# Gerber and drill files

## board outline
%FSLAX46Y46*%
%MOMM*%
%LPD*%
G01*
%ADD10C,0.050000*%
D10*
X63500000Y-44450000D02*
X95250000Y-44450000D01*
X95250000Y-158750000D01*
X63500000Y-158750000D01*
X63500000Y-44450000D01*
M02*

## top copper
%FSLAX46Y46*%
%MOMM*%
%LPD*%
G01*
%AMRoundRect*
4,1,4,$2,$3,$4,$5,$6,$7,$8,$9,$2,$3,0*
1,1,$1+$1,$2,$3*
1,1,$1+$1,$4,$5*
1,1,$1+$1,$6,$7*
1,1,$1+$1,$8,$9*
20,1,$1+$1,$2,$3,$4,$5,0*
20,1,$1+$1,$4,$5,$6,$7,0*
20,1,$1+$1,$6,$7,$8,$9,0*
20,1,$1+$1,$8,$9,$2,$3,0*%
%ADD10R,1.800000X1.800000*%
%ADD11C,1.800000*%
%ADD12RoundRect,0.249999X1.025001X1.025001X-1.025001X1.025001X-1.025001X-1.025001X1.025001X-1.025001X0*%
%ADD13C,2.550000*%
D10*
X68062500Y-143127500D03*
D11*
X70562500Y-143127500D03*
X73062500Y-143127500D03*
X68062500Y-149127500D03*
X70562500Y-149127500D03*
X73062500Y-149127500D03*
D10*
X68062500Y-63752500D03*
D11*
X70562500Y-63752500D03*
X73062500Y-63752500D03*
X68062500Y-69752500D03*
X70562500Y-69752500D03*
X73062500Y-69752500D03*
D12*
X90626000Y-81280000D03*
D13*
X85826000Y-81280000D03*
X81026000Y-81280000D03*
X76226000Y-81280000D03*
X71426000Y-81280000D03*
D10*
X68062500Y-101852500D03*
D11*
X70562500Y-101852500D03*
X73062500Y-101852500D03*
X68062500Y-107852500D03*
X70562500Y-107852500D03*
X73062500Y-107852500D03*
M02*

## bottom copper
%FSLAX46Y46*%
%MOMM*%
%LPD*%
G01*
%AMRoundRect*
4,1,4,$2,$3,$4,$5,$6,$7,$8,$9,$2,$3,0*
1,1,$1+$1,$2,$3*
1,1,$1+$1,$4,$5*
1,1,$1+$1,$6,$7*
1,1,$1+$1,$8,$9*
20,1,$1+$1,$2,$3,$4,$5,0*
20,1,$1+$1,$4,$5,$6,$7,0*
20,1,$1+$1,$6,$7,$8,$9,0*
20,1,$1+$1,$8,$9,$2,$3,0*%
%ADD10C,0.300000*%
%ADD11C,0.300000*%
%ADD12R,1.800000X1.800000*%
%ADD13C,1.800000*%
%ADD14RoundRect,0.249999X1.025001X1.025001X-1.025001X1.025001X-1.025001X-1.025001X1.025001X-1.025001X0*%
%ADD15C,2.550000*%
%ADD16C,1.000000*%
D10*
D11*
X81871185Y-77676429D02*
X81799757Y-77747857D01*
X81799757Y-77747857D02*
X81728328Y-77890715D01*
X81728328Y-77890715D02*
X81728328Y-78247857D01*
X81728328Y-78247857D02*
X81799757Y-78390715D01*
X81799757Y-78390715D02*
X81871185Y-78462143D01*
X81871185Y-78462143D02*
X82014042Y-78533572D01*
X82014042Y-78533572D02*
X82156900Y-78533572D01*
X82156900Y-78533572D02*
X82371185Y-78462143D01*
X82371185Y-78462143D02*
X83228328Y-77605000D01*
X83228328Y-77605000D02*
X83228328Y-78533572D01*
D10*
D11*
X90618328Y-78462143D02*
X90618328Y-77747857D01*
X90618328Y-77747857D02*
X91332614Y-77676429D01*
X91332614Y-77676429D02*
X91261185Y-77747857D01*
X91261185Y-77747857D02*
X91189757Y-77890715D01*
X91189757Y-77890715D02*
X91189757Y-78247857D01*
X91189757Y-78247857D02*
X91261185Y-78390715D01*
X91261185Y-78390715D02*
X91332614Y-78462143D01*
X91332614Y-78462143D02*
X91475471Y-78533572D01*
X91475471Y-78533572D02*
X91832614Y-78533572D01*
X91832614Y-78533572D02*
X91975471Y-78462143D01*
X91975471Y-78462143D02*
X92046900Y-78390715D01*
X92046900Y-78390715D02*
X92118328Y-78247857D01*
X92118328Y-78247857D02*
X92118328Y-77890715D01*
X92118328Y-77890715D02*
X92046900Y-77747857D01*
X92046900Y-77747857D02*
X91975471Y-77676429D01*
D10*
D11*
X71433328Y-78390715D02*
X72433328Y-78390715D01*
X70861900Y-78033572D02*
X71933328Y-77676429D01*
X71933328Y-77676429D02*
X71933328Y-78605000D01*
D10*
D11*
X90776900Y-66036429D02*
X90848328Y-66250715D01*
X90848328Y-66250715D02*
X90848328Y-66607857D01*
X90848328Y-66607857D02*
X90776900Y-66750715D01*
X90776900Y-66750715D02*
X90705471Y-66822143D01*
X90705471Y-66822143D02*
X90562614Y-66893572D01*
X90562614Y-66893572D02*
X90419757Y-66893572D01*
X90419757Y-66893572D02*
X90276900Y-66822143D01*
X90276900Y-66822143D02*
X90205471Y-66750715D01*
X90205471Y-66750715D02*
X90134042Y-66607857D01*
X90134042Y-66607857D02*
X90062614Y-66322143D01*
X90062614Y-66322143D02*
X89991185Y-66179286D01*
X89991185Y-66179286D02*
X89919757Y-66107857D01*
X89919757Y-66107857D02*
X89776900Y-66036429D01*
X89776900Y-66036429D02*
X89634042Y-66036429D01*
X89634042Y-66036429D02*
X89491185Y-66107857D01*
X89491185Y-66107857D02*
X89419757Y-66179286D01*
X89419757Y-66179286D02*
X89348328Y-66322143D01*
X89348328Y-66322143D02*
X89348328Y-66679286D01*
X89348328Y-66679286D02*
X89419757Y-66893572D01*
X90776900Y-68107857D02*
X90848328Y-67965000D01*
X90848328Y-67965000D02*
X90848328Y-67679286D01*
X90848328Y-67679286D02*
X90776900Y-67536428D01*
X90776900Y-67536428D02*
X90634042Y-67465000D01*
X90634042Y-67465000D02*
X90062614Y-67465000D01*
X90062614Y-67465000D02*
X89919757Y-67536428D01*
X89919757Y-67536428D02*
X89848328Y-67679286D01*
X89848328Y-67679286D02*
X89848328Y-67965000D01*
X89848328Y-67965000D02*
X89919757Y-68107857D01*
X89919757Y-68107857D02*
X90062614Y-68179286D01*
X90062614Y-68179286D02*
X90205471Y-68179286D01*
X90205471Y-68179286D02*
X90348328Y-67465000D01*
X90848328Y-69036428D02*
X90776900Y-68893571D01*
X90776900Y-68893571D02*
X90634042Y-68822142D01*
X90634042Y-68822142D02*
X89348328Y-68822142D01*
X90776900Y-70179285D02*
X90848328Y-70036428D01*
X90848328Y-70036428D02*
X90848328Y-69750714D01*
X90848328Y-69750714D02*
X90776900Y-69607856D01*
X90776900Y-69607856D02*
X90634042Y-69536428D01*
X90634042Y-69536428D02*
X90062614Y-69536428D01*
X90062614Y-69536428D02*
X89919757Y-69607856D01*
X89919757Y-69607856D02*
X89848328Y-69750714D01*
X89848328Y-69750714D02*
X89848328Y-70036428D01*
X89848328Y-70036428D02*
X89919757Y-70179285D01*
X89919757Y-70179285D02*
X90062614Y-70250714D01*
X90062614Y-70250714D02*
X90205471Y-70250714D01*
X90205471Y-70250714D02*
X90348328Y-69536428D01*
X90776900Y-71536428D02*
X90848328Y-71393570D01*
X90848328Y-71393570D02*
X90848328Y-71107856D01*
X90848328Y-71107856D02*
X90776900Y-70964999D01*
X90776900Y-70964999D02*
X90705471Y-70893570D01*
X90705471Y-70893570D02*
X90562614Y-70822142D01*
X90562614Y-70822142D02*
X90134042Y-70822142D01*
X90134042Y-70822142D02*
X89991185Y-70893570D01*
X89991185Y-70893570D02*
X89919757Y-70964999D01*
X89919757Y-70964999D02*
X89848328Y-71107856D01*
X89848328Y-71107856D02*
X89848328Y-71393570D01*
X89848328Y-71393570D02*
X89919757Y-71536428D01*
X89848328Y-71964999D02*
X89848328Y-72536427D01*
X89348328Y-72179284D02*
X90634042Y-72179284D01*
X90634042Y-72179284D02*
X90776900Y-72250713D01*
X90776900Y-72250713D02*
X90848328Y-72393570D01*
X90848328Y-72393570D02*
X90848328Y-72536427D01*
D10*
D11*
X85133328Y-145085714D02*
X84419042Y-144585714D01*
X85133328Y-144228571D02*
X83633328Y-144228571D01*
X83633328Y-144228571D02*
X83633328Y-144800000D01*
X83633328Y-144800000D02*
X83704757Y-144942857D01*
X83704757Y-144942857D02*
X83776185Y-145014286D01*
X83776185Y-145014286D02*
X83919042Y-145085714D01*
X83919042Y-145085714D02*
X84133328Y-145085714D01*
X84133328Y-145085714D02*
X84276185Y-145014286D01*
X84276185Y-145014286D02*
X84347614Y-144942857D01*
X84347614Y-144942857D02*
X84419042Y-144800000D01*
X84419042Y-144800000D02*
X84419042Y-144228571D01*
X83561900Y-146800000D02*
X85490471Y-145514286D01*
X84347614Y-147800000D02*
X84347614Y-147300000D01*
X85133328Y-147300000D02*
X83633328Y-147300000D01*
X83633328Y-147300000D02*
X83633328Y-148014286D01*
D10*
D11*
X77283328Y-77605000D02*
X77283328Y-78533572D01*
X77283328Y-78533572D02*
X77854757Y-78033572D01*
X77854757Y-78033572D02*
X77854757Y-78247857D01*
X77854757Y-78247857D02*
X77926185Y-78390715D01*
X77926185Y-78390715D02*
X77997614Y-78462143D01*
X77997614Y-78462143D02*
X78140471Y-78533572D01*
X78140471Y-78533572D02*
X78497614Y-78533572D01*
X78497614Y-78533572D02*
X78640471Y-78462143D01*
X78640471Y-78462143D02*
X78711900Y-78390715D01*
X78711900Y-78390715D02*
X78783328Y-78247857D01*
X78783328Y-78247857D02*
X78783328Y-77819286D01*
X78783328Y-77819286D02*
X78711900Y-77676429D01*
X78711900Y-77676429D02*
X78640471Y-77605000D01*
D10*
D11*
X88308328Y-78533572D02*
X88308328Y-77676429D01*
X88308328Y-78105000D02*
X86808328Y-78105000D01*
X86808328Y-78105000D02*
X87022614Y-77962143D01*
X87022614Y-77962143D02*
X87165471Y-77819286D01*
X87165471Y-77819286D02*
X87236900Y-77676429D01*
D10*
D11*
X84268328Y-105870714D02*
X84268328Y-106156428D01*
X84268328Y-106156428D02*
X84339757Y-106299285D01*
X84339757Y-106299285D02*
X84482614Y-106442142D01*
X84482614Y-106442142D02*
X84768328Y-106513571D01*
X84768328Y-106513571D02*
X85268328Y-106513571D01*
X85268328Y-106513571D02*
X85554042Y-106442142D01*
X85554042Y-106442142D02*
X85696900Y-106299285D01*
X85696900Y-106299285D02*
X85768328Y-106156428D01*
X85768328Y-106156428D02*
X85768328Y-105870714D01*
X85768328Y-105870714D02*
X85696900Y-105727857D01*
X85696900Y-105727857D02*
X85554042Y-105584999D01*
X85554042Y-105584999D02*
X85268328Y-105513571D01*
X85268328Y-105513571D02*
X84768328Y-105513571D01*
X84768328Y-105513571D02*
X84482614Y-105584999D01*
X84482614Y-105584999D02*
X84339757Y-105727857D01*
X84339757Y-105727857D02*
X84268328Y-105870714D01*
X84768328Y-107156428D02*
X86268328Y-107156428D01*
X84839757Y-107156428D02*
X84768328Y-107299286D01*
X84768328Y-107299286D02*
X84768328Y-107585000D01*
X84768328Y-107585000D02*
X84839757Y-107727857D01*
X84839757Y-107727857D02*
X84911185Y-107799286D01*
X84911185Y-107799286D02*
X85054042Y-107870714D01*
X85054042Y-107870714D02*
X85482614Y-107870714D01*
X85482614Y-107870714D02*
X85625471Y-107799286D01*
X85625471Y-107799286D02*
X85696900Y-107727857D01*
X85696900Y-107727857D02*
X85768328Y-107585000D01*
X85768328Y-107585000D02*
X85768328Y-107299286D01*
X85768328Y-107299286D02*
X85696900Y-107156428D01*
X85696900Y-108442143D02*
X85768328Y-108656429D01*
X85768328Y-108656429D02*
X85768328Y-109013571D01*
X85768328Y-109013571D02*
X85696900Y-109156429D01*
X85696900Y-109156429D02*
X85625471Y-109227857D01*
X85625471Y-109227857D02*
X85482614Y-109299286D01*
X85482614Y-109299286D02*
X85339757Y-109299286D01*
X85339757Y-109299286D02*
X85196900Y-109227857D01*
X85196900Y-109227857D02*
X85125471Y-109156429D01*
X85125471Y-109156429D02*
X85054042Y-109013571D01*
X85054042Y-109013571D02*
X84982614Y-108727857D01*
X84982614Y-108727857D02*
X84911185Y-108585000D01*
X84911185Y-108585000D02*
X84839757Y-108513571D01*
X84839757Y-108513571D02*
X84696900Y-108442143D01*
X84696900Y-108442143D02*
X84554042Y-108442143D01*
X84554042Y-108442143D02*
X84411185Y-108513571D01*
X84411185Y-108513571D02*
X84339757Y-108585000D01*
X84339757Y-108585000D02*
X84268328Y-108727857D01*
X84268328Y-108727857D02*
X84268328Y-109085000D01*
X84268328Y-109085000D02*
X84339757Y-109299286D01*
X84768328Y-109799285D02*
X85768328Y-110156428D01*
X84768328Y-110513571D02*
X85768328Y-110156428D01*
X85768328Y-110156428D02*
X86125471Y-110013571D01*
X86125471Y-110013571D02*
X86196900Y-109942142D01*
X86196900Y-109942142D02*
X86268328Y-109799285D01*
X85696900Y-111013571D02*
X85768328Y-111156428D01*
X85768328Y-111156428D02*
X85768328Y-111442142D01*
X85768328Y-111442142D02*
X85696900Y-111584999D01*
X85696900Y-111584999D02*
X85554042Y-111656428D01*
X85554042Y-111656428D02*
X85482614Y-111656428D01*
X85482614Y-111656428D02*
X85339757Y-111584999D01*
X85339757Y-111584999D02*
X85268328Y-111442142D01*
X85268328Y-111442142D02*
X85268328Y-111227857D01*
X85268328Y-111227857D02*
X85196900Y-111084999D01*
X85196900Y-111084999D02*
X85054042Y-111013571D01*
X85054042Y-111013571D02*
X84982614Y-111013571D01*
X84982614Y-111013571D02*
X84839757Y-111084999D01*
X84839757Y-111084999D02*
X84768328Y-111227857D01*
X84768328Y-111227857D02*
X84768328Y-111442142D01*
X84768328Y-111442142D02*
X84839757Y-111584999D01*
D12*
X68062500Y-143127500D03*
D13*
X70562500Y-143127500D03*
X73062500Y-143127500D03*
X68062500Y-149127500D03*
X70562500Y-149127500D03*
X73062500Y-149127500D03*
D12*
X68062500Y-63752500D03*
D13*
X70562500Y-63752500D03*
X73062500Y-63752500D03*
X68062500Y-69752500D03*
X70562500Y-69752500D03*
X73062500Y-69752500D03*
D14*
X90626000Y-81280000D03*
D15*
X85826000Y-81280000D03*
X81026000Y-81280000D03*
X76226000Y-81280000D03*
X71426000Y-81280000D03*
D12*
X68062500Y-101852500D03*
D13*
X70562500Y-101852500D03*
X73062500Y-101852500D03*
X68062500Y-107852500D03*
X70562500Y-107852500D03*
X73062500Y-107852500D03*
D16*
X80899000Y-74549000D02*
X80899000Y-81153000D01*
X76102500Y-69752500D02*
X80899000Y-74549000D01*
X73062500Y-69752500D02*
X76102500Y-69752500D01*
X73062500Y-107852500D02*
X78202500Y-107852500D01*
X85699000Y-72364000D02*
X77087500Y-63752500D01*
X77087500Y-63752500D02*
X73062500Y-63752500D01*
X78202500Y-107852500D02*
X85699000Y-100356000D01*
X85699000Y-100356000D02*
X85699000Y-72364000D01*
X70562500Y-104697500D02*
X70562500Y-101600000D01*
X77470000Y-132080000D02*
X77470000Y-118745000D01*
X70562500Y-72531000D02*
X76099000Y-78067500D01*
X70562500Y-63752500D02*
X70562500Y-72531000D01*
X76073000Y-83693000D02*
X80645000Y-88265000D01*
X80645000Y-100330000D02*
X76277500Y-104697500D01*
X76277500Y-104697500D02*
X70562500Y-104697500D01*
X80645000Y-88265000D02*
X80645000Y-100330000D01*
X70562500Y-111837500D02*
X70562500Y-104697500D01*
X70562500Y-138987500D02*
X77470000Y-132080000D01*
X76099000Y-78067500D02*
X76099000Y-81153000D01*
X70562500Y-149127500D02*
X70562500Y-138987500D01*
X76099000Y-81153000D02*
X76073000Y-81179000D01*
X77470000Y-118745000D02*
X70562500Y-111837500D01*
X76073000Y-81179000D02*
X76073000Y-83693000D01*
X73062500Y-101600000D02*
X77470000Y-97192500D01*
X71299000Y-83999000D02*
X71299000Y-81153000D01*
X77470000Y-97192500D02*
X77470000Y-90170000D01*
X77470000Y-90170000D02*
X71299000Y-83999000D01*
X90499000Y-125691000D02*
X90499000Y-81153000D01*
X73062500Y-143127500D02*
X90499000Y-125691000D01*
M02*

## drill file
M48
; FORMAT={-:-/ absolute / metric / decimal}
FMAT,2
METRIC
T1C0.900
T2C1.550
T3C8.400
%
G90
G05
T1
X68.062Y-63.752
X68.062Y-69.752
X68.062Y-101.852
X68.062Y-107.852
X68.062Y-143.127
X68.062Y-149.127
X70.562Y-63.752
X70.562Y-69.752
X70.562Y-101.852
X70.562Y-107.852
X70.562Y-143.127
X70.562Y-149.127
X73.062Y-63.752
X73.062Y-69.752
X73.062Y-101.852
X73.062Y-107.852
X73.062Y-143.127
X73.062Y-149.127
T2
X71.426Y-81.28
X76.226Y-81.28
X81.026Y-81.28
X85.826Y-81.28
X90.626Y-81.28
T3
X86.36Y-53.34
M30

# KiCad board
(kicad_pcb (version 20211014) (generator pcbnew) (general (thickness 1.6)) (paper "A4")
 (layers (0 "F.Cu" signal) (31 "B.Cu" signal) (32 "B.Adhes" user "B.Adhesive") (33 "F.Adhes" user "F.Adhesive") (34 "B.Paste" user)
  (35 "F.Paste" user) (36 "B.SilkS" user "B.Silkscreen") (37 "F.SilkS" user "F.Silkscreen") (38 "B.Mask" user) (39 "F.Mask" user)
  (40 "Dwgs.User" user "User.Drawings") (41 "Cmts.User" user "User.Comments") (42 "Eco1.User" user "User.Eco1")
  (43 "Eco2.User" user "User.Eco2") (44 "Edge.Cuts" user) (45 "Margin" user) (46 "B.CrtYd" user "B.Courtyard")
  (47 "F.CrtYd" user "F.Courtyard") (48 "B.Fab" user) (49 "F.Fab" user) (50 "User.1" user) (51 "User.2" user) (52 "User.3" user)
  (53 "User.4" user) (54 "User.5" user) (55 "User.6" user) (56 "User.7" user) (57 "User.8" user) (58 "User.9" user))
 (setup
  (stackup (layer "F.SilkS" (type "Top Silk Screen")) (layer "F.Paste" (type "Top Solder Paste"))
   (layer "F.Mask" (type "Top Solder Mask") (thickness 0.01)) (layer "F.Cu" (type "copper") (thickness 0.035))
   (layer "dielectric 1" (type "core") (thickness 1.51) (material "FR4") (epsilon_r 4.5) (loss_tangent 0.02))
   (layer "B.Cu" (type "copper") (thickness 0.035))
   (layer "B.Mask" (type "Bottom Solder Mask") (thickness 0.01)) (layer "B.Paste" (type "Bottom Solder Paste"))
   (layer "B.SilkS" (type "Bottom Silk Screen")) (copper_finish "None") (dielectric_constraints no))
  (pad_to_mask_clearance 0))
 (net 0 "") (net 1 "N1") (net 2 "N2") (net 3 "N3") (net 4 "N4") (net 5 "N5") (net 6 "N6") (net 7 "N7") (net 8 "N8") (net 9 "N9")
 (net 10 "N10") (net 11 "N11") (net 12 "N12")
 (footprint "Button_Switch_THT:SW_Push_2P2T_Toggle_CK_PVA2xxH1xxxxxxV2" (layer "F.Cu") (at 68.0625 143.1275)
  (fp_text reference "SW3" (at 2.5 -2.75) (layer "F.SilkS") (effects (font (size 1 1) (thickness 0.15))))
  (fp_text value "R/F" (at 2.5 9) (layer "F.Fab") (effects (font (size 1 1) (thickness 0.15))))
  (pad "1" thru_hole rect (at 0 0) (size 1.8 1.8) (drill 0.9) (layers *.Cu *.Mask) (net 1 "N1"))
  (pad "2" thru_hole circle (at 2.5 0) (size 1.8 1.8) (drill 0.9) (layers *.Cu *.Mask) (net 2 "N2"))
  (pad "3" thru_hole circle (at 5 0) (size 1.8 1.8) (drill 0.9) (layers *.Cu *.Mask) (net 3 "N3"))
  (pad "4" thru_hole circle (at 0 6) (size 1.8 1.8) (drill 0.9) (layers *.Cu *.Mask) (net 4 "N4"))
  (pad "5" thru_hole circle (at 2.5 6) (size 1.8 1.8) (drill 0.9) (layers *.Cu *.Mask) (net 2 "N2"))
  (pad "6" thru_hole circle (at 5 6) (size 1.8 1.8) (drill 0.9) (layers *.Cu *.Mask) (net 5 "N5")))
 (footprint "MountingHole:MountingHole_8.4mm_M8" (layer "F.Cu") (at 86.36 53.34)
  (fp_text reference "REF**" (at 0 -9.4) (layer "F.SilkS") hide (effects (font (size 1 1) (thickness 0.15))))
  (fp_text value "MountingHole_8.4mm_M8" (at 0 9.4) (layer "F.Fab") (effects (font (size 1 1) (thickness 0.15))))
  (pad "" np_thru_hole circle (at 0 0) (size 8.4 8.4) (drill 8.4) (layers *.Cu *.Mask)))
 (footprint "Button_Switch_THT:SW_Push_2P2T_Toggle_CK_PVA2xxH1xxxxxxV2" (layer "F.Cu") (at 68.0625 63.7525)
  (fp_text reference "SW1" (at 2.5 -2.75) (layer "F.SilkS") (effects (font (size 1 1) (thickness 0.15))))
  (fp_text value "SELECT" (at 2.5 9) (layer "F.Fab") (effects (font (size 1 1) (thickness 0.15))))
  (pad "1" thru_hole rect (at 0 0) (size 1.8 1.8) (drill 0.9) (layers *.Cu *.Mask) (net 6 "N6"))
  (pad "2" thru_hole circle (at 2.5 0) (size 1.8 1.8) (drill 0.9) (layers *.Cu *.Mask) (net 2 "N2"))
  (pad "3" thru_hole circle (at 5 0) (size 1.8 1.8) (drill 0.9) (layers *.Cu *.Mask) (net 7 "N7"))
  (pad "4" thru_hole circle (at 0 6) (size 1.8 1.8) (drill 0.9) (layers *.Cu *.Mask) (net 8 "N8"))
  (pad "5" thru_hole circle (at 2.5 6) (size 1.8 1.8) (drill 0.9) (layers *.Cu *.Mask) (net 2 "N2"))
  (pad "6" thru_hole circle (at 5 6) (size 1.8 1.8) (drill 0.9) (layers *.Cu *.Mask) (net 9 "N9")))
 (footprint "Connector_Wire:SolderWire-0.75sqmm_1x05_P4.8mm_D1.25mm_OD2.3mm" (layer "F.Cu") (at 90.626 81.28 180)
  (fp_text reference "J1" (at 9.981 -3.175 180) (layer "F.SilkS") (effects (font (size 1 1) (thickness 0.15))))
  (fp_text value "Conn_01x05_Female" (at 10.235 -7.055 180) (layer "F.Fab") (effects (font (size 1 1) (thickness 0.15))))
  (pad "1" thru_hole roundrect (at 0 0 180) (size 2.55 2.55) (drill 1.55) (layers *.Cu *.Mask) (roundrect_rratio 0.098039) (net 3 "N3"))
  (pad "2" thru_hole circle (at 4.8 0 180) (size 2.55 2.55) (drill 1.55) (layers *.Cu *.Mask) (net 7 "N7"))
  (pad "3" thru_hole circle (at 9.6 0 180) (size 2.55 2.55) (drill 1.55) (layers *.Cu *.Mask) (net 9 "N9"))
  (pad "4" thru_hole circle (at 14.4 0 180) (size 2.55 2.55) (drill 1.55) (layers *.Cu *.Mask) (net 2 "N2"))
  (pad "5" thru_hole circle (at 19.2 0 180) (size 2.55 2.55) (drill 1.55) (layers *.Cu *.Mask) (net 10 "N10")))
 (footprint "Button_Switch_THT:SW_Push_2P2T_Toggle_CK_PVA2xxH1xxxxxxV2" (layer "F.Cu") (at 68.0625 101.8525)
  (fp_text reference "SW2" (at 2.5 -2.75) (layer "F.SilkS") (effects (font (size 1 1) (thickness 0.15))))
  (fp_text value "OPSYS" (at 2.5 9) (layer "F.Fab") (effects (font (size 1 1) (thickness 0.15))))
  (pad "1" thru_hole rect (at 0 0) (size 1.8 1.8) (drill 0.9) (layers *.Cu *.Mask) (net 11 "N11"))
  (pad "2" thru_hole circle (at 2.5 0) (size 1.8 1.8) (drill 0.9) (layers *.Cu *.Mask) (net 2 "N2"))
  (pad "3" thru_hole circle (at 5 0) (size 1.8 1.8) (drill 0.9) (layers *.Cu *.Mask) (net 10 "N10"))
  (pad "4" thru_hole circle (at 0 6) (size 1.8 1.8) (drill 0.9) (layers *.Cu *.Mask) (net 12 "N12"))
  (pad "5" thru_hole circle (at 2.5 6) (size 1.8 1.8) (drill 0.9) (layers *.Cu *.Mask) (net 2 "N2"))
  (pad "6" thru_hole circle (at 5 6) (size 1.8 1.8) (drill 0.9) (layers *.Cu *.Mask) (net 7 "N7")))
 (gr_rect (start 63.5 44.45) (end 95.25 158.75) (layer "Edge.Cuts") (width 0.05) (fill none))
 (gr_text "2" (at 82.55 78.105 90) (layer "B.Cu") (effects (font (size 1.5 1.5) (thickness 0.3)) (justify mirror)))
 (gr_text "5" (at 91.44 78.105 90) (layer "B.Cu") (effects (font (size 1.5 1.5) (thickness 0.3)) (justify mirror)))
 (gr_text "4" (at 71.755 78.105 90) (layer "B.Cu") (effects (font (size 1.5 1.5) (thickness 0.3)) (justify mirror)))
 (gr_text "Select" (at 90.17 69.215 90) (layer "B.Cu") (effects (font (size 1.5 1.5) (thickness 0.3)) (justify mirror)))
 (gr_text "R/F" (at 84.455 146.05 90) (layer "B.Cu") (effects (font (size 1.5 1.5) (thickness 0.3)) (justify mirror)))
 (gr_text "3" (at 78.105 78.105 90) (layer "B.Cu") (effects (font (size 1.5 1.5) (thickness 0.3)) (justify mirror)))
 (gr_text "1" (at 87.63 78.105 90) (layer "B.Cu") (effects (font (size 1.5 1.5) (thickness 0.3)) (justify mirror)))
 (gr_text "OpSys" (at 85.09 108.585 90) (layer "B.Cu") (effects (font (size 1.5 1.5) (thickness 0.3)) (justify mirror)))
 (segment (start 80.899 74.549) (end 80.899 81.153) (width 1) (layer "B.Cu") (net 9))
 (segment (start 76.1025 69.7525) (end 80.899 74.549) (width 1) (layer "B.Cu") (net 9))
 (segment (start 73.0625 69.7525) (end 76.1025 69.7525) (width 1) (layer "B.Cu") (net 9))
 (segment (start 73.0625 107.8525) (end 78.2025 107.8525) (width 1) (layer "B.Cu") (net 7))
 (segment (start 85.699 72.364) (end 77.0875 63.7525) (width 1) (layer "B.Cu") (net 7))
 (segment (start 77.0875 63.7525) (end 73.0625 63.7525) (width 1) (layer "B.Cu") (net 7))
 (segment (start 78.2025 107.8525) (end 85.699 100.356) (width 1) (layer "B.Cu") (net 7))
 (segment (start 85.699 100.356) (end 85.699 72.364) (width 1) (layer "B.Cu") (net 7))
 (segment (start 70.5625 104.6975) (end 70.5625 101.6) (width 1) (layer "B.Cu") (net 2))
 (segment (start 77.47 132.08) (end 77.47 118.745) (width 1) (layer "B.Cu") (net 2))
 (segment (start 70.5625 72.531) (end 76.099 78.0675) (width 1) (layer "B.Cu") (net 2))
 (segment (start 70.5625 63.7525) (end 70.5625 72.531) (width 1) (layer "B.Cu") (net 2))
 (segment (start 76.073 83.693) (end 80.645 88.265) (width 1) (layer "B.Cu") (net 2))
 (segment (start 80.645 100.33) (end 76.2775 104.6975) (width 1) (layer "B.Cu") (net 2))
 (segment (start 76.2775 104.6975) (end 70.5625 104.6975) (width 1) (layer "B.Cu") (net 2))
 (segment (start 80.645 88.265) (end 80.645 100.33) (width 1) (layer "B.Cu") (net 2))
 (segment (start 70.5625 111.8375) (end 70.5625 104.6975) (width 1) (layer "B.Cu") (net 2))
 (segment (start 70.5625 138.9875) (end 77.47 132.08) (width 1) (layer "B.Cu") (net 2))
 (segment (start 76.099 78.0675) (end 76.099 81.153) (width 1) (layer "B.Cu") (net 2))
 (segment (start 70.5625 149.1275) (end 70.5625 138.9875) (width 1) (layer "B.Cu") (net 2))
 (segment (start 76.099 81.153) (end 76.073 81.179) (width 1) (layer "B.Cu") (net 2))
 (segment (start 77.47 118.745) (end 70.5625 111.8375) (width 1) (layer "B.Cu") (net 2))
 (segment (start 76.073 81.179) (end 76.073 83.693) (width 1) (layer "B.Cu") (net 2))
 (segment (start 73.0625 101.6) (end 77.47 97.1925) (width 1) (layer "B.Cu") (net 10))
 (segment (start 71.299 83.999) (end 71.299 81.153) (width 1) (layer "B.Cu") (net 10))
 (segment (start 77.47 97.1925) (end 77.47 90.17) (width 1) (layer "B.Cu") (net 10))
 (segment (start 77.47 90.17) (end 71.299 83.999) (width 1) (layer "B.Cu") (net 10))
 (segment (start 90.499 125.691) (end 90.499 81.153) (width 1) (layer "B.Cu") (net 3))
 (segment (start 73.0625 143.1275) (end 90.499 125.691) (width 1) (layer "B.Cu") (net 3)))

